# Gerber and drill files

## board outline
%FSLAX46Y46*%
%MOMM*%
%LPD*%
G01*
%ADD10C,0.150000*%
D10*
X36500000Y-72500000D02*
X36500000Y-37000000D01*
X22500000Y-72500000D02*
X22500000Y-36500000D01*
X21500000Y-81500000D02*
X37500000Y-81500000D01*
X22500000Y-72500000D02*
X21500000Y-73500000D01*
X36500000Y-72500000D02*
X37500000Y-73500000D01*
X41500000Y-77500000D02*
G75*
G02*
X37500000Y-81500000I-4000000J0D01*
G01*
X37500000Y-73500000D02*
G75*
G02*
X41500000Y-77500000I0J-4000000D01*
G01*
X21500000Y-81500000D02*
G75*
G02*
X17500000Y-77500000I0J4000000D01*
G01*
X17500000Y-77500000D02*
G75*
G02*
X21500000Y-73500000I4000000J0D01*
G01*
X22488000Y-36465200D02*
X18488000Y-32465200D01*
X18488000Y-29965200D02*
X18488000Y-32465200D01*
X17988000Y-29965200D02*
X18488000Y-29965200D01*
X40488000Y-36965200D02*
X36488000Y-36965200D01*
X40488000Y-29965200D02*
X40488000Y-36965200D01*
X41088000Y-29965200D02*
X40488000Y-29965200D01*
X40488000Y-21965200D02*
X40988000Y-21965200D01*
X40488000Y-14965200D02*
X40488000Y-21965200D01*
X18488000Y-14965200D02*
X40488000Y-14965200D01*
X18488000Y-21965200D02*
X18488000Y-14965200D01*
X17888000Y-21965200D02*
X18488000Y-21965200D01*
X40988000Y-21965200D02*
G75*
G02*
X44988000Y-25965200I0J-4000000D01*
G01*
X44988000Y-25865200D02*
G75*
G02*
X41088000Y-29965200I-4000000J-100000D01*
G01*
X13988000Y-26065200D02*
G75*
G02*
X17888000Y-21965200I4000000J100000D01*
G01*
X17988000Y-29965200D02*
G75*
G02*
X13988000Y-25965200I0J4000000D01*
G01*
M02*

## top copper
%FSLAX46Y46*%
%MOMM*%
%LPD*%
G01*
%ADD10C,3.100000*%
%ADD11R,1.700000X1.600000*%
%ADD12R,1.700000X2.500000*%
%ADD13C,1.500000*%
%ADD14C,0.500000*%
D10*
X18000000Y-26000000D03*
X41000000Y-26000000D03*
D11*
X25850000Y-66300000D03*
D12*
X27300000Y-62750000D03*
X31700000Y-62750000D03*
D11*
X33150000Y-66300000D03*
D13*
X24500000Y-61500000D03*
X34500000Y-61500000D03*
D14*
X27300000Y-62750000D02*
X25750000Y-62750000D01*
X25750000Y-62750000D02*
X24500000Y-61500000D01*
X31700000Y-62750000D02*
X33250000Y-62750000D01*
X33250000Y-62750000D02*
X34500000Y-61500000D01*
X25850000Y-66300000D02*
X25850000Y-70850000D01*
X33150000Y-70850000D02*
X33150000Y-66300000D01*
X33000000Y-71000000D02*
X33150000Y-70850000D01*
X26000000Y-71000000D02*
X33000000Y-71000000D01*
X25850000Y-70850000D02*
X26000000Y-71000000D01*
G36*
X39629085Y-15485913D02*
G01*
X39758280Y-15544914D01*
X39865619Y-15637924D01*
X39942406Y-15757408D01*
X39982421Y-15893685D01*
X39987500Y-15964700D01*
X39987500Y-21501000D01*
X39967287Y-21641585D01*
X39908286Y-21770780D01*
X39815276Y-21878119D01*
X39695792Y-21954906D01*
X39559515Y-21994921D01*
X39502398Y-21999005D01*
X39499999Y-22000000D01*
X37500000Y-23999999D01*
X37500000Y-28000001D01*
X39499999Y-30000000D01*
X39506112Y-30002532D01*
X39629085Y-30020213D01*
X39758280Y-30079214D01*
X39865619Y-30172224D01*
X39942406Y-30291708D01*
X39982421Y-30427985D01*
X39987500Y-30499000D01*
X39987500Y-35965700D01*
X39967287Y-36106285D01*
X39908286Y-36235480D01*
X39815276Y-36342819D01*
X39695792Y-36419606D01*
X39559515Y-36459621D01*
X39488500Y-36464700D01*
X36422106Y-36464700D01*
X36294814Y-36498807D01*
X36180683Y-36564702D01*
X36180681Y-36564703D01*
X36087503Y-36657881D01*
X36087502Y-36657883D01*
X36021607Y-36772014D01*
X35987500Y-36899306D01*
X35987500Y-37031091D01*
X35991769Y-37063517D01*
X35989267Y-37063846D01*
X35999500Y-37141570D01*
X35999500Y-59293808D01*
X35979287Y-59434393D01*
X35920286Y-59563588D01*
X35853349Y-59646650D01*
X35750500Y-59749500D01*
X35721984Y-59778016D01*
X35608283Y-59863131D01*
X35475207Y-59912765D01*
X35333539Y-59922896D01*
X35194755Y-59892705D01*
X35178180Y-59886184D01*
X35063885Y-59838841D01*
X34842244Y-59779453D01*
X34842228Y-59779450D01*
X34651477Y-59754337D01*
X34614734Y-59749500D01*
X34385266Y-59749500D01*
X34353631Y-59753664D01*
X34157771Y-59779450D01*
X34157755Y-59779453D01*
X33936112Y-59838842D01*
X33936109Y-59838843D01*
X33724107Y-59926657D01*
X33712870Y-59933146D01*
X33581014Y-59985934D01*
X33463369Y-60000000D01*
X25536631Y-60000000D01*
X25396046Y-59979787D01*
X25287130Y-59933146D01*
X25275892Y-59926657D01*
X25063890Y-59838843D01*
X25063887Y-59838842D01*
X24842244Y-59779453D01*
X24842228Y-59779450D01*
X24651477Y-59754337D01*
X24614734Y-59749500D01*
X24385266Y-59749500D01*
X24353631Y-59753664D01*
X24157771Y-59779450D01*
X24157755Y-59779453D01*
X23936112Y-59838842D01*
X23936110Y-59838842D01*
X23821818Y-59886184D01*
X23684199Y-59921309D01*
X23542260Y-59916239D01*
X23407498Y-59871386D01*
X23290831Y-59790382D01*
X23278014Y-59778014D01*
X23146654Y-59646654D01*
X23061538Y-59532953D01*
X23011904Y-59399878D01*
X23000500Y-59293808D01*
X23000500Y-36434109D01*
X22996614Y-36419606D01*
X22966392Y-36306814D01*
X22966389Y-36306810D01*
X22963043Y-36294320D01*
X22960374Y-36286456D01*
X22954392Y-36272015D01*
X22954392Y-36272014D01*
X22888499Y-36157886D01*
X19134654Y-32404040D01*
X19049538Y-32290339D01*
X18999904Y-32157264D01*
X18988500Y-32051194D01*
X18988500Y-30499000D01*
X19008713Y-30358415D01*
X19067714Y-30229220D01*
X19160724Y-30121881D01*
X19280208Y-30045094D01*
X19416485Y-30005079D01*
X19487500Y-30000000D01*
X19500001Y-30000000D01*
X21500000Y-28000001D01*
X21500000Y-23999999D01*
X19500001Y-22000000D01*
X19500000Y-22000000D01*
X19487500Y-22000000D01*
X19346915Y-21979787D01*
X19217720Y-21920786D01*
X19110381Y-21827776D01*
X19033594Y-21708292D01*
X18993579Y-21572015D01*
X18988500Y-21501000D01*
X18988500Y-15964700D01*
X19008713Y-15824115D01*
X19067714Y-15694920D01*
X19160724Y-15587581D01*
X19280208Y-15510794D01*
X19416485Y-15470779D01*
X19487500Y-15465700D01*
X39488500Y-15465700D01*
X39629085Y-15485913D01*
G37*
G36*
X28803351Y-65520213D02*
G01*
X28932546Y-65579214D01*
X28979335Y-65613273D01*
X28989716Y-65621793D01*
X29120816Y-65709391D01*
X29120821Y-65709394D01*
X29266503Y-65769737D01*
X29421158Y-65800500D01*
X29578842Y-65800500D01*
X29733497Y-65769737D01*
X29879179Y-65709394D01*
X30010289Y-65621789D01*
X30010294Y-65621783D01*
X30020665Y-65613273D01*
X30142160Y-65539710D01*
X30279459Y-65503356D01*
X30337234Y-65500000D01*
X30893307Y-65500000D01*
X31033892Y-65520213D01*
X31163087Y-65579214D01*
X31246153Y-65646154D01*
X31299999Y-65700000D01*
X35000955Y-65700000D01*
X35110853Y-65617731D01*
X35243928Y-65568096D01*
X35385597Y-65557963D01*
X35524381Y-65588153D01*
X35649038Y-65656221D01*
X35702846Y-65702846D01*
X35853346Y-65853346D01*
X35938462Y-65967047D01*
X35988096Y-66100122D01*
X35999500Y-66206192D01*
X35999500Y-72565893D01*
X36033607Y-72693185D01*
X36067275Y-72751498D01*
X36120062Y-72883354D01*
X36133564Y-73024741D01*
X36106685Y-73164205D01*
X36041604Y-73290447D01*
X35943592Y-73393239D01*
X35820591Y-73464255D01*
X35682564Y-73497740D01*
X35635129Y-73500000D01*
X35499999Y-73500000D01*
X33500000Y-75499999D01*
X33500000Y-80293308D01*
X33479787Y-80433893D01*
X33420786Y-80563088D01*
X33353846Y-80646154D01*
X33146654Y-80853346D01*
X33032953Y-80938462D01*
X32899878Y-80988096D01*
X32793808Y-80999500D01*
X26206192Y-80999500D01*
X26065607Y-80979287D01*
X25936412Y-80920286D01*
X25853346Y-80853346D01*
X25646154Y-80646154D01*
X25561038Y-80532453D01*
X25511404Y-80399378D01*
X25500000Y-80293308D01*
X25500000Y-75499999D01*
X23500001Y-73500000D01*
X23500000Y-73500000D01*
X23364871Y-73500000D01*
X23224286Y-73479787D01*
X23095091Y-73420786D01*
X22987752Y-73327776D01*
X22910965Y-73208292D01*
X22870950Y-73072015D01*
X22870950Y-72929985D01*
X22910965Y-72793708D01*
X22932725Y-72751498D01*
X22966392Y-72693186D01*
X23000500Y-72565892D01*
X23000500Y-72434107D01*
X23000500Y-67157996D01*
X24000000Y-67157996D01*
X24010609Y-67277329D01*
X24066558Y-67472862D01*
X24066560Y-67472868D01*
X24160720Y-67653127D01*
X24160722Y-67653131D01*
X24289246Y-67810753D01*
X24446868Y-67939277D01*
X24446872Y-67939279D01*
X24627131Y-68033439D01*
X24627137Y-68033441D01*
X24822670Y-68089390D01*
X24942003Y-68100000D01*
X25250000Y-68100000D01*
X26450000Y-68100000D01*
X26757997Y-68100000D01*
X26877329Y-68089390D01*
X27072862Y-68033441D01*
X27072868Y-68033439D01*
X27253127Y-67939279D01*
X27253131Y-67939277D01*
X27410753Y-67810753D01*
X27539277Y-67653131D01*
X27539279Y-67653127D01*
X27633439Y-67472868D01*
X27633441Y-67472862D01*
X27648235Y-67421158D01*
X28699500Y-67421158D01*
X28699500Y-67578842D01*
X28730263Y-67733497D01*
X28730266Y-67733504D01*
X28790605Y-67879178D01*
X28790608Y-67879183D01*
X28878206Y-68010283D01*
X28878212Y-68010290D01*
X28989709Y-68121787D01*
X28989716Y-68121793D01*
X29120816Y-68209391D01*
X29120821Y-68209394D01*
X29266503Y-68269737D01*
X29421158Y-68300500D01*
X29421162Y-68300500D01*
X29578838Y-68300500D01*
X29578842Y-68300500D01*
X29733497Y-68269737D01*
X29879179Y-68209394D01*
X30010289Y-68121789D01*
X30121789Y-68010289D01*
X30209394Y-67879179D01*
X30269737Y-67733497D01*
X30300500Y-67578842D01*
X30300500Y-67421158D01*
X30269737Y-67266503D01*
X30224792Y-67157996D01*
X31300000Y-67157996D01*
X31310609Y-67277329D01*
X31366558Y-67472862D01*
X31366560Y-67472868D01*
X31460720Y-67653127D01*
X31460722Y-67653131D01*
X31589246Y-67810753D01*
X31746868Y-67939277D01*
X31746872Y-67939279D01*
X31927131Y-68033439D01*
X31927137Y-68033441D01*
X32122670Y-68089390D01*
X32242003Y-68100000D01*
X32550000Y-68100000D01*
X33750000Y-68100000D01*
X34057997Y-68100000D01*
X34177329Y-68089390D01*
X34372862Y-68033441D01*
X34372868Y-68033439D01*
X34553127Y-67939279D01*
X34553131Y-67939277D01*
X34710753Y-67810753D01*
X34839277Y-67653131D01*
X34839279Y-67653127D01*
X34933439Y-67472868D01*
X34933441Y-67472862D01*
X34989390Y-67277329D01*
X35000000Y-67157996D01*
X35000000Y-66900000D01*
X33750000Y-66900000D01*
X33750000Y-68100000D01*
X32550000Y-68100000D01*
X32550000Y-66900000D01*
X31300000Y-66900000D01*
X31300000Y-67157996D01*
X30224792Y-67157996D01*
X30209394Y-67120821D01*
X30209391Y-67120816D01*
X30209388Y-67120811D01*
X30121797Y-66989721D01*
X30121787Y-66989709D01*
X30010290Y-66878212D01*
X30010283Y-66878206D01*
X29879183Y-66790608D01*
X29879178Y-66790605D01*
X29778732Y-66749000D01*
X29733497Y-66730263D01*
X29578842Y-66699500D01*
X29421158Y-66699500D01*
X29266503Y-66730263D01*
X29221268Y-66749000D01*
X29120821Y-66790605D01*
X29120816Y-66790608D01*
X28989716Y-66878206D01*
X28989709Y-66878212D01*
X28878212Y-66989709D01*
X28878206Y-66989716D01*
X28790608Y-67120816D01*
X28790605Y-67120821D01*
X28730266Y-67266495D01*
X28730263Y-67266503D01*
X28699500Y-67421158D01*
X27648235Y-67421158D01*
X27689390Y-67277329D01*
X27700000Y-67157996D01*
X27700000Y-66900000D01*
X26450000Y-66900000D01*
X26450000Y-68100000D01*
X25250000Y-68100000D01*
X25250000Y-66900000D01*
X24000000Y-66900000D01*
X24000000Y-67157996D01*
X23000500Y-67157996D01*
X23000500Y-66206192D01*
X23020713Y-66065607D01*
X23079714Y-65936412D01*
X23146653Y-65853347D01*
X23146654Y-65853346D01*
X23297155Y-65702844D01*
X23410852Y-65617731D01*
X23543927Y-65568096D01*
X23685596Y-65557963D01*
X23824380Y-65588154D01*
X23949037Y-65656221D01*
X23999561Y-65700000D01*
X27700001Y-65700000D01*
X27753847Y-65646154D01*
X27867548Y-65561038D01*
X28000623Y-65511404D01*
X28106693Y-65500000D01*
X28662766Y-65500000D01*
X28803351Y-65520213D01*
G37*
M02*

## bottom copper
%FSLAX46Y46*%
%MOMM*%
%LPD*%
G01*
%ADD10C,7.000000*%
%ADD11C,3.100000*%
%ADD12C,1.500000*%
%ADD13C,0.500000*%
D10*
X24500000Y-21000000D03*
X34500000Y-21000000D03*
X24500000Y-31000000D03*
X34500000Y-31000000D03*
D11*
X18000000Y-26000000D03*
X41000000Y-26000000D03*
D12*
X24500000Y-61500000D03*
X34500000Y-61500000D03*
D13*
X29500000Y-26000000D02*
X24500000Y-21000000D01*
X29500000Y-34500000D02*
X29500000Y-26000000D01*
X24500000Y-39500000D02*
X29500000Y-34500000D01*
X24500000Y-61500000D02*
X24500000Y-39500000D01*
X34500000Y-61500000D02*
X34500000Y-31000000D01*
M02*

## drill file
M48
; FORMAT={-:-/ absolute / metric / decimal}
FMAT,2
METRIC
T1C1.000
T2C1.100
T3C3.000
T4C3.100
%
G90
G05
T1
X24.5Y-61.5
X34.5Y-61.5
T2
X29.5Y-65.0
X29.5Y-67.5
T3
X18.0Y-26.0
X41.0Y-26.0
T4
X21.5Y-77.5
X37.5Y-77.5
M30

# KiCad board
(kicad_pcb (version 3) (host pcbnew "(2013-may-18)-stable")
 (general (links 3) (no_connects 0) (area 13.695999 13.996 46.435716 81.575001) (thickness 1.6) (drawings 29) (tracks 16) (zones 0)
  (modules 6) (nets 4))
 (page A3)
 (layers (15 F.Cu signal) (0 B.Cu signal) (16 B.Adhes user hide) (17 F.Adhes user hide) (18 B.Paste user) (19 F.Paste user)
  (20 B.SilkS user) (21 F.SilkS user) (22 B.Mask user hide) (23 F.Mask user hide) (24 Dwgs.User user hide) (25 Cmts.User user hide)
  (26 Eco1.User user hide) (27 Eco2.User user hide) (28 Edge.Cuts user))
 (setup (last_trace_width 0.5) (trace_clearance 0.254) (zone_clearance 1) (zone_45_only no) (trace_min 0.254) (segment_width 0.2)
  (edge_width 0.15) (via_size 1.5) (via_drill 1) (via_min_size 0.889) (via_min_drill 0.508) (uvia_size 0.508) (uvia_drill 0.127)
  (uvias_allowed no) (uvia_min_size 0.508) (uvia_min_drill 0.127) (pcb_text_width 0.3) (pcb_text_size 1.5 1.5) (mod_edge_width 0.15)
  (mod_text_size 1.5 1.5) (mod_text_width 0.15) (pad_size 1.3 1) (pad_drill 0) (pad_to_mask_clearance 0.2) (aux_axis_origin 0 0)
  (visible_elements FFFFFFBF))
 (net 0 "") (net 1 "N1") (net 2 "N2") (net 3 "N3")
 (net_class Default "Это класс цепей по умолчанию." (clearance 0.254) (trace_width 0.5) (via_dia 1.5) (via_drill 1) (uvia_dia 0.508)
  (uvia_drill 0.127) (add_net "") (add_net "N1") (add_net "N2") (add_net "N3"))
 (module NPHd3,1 (layer F.Cu) (at 21.5 76.5)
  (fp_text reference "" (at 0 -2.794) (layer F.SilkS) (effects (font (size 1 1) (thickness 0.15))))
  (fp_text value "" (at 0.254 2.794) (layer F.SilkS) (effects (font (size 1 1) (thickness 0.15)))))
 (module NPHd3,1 (layer F.Cu) (at 37.5 76.5)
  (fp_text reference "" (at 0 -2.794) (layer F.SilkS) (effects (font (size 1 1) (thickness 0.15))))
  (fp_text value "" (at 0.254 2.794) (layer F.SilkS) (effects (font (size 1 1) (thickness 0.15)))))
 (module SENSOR (layer B.Cu) (at 18 14.5)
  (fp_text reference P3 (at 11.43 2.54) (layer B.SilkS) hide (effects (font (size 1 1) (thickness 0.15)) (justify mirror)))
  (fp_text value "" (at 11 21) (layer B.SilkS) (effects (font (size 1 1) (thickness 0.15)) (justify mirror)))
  (pad 2 smd circle (at 6.5 6.5) (size 7 7) (layers B.Cu B.Mask) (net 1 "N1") (solder_mask_margin 0.1))
  (pad 3 smd circle (at 16.5 6.5) (size 7 7) (layers B.Cu B.Mask))
  (pad 1 smd circle (at 6.5 16.5) (size 7 7) (layers B.Cu B.Mask))
  (pad 4 smd circle (at 16.5 16.5) (size 7 7) (layers B.Cu B.Mask) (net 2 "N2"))
  (pad "" np_thru_hole circle (at 0 11.5) (size 3.1 3.1) (drill 3) (layers *.Cu *.Mask B.SilkS))
  (pad "" np_thru_hole circle (at 23 11.5) (size 3.1 3.1) (drill 3) (layers *.Cu *.Mask B.SilkS)))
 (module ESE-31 (layer F.Cu) (at 29.5 62.75 180)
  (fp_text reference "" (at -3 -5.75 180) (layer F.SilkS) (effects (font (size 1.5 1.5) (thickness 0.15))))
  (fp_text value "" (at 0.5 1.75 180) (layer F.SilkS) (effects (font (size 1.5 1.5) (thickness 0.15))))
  (pad "" np_thru_hole circle (at 0 -4.75 180) (size 1.1 1.1) (drill 1.1) (layers *.Cu *.Mask F.SilkS))
  (pad 4 smd rect (at 3.65 -3.55 180) (size 1.7 1.6) (layers F.Cu F.Paste F.Mask) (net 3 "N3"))
  (pad 2 smd rect (at 2.2 0 180) (size 1.7 2.5) (layers F.Cu F.Paste F.Mask) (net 1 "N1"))
  (pad 1 smd rect (at -2.2 0 180) (size 1.7 2.5) (layers F.Cu F.Paste F.Mask) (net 2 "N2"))
  (pad 3 smd rect (at -3.65 -3.55 180) (size 1.7 1.6) (layers F.Cu F.Paste F.Mask) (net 3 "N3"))
  (pad "" np_thru_hole circle (at 0 -2.25 180) (size 1.1 1.1) (drill 1.1) (layers *.Cu *.Mask F.SilkS)))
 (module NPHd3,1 (layer F.Cu) (at 21.5 77.5)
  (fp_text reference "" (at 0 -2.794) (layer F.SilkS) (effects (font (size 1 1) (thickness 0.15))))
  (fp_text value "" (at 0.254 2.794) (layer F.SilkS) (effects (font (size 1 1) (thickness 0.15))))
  (pad "" np_thru_hole circle (at 0 0) (size 3.1 3.1) (drill 3.1) (layers *.Cu *.Mask F.SilkS)))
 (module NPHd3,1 (layer F.Cu) (at 37.5 77.5)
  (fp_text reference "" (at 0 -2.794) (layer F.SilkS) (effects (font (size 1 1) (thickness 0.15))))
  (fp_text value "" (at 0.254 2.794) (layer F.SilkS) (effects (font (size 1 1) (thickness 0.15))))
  (pad "" np_thru_hole circle (at 0 0) (size 3.1 3.1) (drill 3.1) (layers *.Cu *.Mask F.SilkS)))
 (gr_line (start 36.5 72.5) (end 36.5 37) (angle 90) (layer Edge.Cuts) (width 0.15))
 (gr_line (start 22.5 72.5) (end 22.5 36.5) (angle 90) (layer Edge.Cuts) (width 0.15))
 (gr_line (start 21.5 81.5) (end 37.5 81.5) (angle 90) (layer Edge.Cuts) (width 0.15))
 (gr_line (start 22.5 72.5) (end 21.5 73.5) (angle 90) (layer Edge.Cuts) (width 0.15))
 (gr_line (start 36.5 72.5) (end 37.5 73.5) (angle 90) (layer Edge.Cuts) (width 0.15))
 (gr_arc (start 37.5 77.5) (end 41.5 77.5) (angle 90) (layer Edge.Cuts) (width 0.15))
 (gr_arc (start 37.5 77.5) (end 37.5 73.5) (angle 90) (layer Edge.Cuts) (width 0.15))
 (gr_arc (start 21.5 77.5) (end 21.5 81.5) (angle 90) (layer Edge.Cuts) (width 0.15))
 (gr_arc (start 21.5 77.5) (end 17.5 77.5) (angle 90) (layer Edge.Cuts) (width 0.15))
 (gr_line (start 22.488 36.4652) (end 18.488 32.4652) (angle 90) (layer Edge.Cuts) (width 0.15))
 (gr_line (start 18.488 29.9652) (end 18.488 32.4652) (angle 90) (layer Edge.Cuts) (width 0.15))
 (gr_line (start 17.988 29.9652) (end 18.488 29.9652) (angle 90) (layer Edge.Cuts) (width 0.15))
 (gr_line (start 40.488 36.9652) (end 36.488 36.9652) (angle 90) (layer Edge.Cuts) (width 0.15))
 (gr_line (start 40.488 29.9652) (end 40.488 36.9652) (angle 90) (layer Edge.Cuts) (width 0.15))
 (gr_line (start 41.088 29.9652) (end 40.488 29.9652) (angle 90) (layer Edge.Cuts) (width 0.15))
 (gr_line (start 40.488 21.9652) (end 40.988 21.9652) (angle 90) (layer Edge.Cuts) (width 0.15))
 (gr_line (start 40.488 14.9652) (end 40.488 21.9652) (angle 90) (layer Edge.Cuts) (width 0.15))
 (gr_line (start 18.488 14.9652) (end 40.488 14.9652) (angle 90) (layer Edge.Cuts) (width 0.15))
 (gr_line (start 18.488 21.9652) (end 18.488 14.9652) (angle 90) (layer Edge.Cuts) (width 0.15))
 (gr_line (start 17.888 21.9652) (end 18.488 21.9652) (angle 90) (layer Edge.Cuts) (width 0.15))
 (gr_arc (start 40.988 25.9652) (end 44.988 25.9652) (angle -90) (layer Edge.Cuts) (width 0.15))
 (gr_arc (start 40.988 25.9652) (end 41.088 29.9652) (angle -90) (layer Edge.Cuts) (width 0.15))
 (gr_arc (start 17.988 25.9652) (end 17.888 21.9652) (angle -90) (layer Edge.Cuts) (width 0.15))
 (gr_arc (start 17.988 25.9652) (end 13.988 25.9652) (angle -90) (layer Edge.Cuts) (width 0.15))
 (segment (start 27.3 62.75) (end 25.75 62.75) (width 0.5) (layer F.Cu) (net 1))
 (segment (start 29.5 26) (end 24.5 21) (width 0.5) (layer B.Cu) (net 1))
 (segment (start 29.5 34.5) (end 29.5 26) (width 0.5) (layer B.Cu) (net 1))
 (segment (start 24.5 39.5) (end 29.5 34.5) (width 0.5) (layer B.Cu) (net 1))
 (segment (start 24.5 61.5) (end 24.5 39.5) (width 0.5) (layer B.Cu) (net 1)) (via (at 24.5 61.5) (size 1.5) (layers F.Cu B.Cu) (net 1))
 (segment (start 25.75 62.75) (end 24.5 61.5) (width 0.5) (layer F.Cu) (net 1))
 (segment (start 31.7 62.75) (end 33.25 62.75) (width 0.5) (layer F.Cu) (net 2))
 (segment (start 34.5 61.5) (end 34.5 31) (width 0.5) (layer B.Cu) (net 2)) (via (at 34.5 61.5) (size 1.5) (layers F.Cu B.Cu) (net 2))
 (segment (start 33.25 62.75) (end 34.5 61.5) (width 0.5) (layer F.Cu) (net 2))
 (segment (start 25.85 66.3) (end 25.85 70.85) (width 0.5) (layer F.Cu) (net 3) (status 400000))
 (segment (start 33.15 70.85) (end 33.15 66.3) (width 0.5) (layer F.Cu) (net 3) (status 800000))
 (segment (start 33 71) (end 33.15 70.85) (width 0.5) (layer F.Cu) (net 3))
 (segment (start 26 71) (end 33 71) (width 0.5) (layer F.Cu) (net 3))
 (segment (start 25.85 70.85) (end 26 71) (width 0.5) (layer F.Cu) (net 3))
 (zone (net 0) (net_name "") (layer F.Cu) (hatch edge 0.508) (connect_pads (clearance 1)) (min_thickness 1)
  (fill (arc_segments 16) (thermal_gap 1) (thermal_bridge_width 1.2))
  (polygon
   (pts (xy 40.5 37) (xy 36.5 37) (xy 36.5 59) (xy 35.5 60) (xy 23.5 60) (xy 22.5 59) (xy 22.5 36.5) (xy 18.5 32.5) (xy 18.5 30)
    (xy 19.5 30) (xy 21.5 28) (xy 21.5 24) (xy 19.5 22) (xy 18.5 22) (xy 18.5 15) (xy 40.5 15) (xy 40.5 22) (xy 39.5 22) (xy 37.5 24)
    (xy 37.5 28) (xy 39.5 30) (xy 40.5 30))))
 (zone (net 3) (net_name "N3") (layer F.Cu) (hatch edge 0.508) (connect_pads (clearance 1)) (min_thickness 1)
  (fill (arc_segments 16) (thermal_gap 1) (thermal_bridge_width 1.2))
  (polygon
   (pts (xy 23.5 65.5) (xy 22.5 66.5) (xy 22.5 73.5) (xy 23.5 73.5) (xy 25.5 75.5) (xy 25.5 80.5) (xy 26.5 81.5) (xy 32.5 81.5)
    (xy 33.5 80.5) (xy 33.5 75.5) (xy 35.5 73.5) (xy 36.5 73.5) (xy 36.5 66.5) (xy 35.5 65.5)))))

